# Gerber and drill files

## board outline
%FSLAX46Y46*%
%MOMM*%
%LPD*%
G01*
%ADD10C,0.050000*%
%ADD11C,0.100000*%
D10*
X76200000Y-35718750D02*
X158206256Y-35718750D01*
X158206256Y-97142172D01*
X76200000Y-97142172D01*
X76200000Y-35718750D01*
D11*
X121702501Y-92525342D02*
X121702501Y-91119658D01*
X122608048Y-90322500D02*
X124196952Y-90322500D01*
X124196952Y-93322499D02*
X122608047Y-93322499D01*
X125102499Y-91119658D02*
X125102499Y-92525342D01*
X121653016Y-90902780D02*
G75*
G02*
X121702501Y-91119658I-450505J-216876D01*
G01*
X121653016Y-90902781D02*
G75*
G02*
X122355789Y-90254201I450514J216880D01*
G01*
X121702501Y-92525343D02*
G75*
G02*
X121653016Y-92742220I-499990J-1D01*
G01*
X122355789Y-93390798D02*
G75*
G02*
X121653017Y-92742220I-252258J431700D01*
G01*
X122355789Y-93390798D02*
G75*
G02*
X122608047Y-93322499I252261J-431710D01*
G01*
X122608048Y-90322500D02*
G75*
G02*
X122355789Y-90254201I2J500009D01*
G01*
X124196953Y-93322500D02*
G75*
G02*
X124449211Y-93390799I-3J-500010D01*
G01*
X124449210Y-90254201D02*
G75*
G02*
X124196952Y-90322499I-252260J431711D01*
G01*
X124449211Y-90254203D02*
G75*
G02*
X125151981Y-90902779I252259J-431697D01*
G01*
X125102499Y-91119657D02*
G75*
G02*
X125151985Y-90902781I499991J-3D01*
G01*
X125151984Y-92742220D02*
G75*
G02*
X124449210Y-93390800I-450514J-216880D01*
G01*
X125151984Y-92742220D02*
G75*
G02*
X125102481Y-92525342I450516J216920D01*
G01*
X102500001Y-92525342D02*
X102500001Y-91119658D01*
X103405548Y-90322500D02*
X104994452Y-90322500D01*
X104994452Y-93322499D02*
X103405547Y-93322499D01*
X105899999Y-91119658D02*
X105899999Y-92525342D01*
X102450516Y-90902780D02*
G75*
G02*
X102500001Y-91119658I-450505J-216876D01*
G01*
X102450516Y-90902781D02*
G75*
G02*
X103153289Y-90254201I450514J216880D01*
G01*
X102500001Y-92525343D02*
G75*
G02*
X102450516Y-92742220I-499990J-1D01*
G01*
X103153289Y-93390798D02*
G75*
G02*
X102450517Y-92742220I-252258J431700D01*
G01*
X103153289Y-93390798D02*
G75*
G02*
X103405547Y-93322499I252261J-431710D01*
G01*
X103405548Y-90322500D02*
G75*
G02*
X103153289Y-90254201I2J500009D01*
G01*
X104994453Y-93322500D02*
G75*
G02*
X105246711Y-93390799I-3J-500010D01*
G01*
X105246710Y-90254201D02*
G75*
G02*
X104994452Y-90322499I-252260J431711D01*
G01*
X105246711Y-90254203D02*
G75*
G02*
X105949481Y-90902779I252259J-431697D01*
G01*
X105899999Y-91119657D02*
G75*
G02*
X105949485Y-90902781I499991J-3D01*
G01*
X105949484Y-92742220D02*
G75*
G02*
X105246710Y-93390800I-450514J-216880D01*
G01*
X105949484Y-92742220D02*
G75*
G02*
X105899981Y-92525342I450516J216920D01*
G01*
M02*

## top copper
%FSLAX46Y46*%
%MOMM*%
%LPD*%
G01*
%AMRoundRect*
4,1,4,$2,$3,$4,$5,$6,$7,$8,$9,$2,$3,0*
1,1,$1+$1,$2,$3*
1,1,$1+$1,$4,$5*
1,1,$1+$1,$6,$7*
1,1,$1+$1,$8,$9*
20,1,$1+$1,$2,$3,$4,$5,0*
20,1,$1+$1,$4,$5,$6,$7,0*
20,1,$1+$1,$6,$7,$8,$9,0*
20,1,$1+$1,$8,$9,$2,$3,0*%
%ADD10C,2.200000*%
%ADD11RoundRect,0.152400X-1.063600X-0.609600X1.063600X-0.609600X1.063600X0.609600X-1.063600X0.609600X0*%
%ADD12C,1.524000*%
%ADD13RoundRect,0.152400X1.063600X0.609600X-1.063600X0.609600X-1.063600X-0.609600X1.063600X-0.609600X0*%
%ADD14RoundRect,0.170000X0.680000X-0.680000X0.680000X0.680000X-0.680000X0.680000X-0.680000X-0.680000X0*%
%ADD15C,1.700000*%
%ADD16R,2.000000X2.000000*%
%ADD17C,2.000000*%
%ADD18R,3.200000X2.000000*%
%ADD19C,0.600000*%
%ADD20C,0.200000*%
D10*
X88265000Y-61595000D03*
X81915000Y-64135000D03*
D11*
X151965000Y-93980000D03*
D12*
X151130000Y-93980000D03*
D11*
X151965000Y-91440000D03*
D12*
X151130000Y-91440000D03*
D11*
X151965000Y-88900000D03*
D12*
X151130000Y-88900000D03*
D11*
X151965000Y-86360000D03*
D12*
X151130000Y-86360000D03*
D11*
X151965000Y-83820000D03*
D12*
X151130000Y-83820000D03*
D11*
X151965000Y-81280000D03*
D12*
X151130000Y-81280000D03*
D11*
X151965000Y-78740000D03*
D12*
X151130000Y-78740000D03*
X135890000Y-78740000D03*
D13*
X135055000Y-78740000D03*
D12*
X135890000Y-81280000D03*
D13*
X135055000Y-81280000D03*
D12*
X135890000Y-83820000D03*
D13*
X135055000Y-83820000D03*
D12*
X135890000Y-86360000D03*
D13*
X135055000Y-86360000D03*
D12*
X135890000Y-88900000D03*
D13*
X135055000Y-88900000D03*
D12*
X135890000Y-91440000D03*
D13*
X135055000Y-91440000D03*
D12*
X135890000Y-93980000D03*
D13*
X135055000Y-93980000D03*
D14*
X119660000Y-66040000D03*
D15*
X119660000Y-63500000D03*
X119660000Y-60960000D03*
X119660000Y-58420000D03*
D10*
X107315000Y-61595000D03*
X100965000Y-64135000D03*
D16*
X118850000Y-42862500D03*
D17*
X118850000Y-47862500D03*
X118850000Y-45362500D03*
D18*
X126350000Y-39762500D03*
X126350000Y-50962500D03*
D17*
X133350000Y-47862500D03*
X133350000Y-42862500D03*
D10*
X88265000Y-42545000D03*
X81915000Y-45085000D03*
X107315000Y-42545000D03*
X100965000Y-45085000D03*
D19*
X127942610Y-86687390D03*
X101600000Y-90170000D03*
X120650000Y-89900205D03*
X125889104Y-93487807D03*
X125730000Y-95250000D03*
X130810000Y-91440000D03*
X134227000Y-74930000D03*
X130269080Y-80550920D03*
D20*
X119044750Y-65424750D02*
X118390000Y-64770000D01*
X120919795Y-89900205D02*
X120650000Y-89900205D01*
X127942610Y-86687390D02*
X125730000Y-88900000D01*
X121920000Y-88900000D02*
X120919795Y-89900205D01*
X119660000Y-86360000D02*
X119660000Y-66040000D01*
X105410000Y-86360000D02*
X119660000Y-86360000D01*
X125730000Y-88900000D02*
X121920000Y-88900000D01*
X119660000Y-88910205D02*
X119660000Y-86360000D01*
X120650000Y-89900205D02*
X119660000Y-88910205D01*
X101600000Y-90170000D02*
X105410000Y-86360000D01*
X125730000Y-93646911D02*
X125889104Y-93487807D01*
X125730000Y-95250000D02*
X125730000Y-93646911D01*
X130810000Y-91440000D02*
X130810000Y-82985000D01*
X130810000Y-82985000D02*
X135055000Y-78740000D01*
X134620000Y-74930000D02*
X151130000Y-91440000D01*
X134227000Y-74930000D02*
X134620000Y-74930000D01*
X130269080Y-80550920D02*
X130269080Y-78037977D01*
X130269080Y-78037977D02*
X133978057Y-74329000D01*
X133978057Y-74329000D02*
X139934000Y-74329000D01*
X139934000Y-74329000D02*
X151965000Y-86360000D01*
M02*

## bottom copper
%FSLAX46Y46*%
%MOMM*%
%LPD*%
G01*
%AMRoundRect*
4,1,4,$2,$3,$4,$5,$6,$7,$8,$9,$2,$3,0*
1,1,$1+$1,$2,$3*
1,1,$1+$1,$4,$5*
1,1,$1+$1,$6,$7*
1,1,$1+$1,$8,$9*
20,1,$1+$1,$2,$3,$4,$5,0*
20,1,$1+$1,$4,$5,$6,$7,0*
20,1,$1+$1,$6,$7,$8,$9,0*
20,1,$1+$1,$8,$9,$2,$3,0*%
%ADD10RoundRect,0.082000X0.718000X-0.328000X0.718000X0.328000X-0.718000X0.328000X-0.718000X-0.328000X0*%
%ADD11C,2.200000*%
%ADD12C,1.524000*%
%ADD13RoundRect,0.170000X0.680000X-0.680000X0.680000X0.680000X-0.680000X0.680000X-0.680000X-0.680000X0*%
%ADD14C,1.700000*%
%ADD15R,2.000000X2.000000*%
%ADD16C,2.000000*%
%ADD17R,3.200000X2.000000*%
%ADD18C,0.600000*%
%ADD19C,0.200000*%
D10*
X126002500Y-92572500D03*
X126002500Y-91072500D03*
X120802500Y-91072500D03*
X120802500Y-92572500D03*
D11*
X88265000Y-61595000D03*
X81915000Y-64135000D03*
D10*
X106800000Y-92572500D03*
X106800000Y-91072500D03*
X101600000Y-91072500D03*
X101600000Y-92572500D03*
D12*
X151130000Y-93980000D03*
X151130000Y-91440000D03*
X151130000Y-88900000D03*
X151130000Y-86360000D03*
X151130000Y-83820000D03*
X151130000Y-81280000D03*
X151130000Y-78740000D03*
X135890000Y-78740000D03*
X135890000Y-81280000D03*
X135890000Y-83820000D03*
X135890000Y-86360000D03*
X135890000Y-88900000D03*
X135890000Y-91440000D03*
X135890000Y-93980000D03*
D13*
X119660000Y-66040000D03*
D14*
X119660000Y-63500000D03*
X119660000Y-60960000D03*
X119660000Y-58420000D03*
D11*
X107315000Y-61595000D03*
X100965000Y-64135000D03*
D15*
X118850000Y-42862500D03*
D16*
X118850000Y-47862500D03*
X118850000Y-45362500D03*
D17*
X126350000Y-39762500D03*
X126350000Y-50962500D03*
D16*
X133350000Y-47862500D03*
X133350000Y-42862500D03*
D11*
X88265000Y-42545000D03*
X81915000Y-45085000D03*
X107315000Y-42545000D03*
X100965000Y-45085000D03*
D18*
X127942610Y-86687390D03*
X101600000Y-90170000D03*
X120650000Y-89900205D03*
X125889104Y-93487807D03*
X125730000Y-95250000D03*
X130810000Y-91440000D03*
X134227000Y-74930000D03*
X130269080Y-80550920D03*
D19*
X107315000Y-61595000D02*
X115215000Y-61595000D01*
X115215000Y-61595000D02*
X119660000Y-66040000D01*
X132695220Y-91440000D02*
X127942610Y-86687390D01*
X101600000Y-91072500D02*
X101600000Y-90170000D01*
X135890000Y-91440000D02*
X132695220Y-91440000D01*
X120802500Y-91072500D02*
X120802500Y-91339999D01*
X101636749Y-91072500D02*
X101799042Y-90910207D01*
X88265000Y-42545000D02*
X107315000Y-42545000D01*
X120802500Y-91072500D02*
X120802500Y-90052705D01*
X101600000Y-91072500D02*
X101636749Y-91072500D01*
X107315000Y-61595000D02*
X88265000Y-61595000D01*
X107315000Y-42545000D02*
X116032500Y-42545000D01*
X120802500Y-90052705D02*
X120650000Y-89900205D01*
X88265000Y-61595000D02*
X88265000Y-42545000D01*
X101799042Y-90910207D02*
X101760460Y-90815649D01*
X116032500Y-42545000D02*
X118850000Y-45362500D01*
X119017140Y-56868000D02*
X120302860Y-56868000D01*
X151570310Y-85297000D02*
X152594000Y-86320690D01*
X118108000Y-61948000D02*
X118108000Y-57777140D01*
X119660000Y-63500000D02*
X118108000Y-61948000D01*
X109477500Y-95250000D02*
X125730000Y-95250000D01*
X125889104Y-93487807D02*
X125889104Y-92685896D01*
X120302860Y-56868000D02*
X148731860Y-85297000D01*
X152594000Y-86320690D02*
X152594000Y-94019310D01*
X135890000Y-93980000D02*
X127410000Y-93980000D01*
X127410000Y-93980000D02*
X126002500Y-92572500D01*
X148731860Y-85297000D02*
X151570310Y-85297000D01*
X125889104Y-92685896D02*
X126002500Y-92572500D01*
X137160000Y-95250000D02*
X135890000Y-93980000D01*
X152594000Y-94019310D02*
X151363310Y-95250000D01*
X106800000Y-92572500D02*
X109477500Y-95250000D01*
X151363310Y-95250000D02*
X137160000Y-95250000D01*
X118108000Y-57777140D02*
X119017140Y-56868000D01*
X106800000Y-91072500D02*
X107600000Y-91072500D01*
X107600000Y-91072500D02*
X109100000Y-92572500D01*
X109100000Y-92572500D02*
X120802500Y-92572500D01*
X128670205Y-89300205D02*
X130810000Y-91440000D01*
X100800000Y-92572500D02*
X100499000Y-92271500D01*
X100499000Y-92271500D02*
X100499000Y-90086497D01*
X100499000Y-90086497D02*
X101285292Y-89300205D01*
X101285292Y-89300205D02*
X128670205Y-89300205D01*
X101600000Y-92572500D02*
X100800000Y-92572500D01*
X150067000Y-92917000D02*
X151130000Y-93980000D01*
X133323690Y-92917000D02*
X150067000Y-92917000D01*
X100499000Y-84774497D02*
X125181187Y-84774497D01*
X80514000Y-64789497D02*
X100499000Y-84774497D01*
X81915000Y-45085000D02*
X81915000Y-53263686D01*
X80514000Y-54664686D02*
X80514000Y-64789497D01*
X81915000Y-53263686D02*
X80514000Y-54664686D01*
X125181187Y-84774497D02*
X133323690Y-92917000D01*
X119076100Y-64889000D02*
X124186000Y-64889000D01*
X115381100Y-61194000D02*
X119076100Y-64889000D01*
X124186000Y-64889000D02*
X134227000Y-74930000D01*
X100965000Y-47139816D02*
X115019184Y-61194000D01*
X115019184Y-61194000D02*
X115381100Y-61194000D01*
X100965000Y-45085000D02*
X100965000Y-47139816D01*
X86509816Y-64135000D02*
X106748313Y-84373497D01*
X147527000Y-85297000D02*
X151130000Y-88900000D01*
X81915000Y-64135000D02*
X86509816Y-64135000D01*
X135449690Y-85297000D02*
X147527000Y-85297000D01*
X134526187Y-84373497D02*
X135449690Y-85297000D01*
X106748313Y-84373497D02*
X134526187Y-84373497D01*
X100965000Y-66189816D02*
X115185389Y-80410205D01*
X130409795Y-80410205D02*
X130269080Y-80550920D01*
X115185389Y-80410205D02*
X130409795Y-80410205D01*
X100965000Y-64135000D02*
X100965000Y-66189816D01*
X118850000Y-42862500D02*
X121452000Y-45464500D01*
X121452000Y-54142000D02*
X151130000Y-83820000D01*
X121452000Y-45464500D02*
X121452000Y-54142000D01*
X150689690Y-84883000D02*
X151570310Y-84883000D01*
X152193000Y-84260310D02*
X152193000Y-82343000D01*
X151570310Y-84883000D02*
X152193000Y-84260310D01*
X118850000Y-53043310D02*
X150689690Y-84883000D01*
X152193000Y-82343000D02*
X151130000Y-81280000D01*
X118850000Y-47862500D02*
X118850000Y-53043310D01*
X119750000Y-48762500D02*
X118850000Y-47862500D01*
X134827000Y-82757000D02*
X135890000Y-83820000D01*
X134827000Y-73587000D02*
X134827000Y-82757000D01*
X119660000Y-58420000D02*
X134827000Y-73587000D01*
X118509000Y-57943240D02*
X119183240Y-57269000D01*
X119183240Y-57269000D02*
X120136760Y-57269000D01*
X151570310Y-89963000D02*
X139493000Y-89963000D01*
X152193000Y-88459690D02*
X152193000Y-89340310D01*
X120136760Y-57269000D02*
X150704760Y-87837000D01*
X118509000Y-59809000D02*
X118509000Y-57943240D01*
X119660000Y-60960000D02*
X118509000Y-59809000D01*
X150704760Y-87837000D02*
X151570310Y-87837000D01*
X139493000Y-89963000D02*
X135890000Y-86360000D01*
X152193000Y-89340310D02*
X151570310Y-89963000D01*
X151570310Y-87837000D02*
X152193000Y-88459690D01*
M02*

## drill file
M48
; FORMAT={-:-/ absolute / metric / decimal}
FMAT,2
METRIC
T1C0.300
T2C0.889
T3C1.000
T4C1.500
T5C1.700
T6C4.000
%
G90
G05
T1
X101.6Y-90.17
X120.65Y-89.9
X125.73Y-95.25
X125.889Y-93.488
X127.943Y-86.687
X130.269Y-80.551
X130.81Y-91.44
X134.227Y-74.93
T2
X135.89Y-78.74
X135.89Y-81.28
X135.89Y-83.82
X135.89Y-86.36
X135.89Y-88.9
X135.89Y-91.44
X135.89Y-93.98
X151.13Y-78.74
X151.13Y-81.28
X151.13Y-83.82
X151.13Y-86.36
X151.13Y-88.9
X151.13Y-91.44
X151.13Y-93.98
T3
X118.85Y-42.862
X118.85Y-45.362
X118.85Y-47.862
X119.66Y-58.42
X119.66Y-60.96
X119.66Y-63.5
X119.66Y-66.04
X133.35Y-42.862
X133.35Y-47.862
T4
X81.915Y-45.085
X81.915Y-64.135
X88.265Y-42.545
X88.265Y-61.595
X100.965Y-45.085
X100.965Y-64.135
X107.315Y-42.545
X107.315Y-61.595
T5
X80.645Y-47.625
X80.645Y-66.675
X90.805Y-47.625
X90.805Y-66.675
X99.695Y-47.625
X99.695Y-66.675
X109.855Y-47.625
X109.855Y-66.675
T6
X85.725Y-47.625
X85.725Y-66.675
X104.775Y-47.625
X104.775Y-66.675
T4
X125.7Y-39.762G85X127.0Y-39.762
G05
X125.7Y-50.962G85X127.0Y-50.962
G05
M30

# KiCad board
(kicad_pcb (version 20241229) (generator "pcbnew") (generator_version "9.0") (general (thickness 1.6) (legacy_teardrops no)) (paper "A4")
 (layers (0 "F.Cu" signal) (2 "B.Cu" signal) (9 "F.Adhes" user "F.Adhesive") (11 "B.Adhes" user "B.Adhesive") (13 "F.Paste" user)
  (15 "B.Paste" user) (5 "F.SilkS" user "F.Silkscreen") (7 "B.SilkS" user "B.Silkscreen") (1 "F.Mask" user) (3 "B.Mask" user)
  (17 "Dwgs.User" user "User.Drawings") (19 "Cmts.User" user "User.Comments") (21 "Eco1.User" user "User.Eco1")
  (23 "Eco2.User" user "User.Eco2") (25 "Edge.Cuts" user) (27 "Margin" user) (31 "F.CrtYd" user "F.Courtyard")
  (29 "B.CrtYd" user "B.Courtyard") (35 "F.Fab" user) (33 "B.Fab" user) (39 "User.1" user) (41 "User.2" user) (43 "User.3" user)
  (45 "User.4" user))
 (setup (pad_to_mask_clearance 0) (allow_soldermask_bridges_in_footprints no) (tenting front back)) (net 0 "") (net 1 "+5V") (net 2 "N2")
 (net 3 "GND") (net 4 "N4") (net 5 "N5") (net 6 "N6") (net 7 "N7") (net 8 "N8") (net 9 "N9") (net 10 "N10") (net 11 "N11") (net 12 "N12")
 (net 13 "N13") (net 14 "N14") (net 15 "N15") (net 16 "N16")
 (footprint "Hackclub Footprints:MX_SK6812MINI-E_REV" (layer "F.Cu") (at 123.4025 86.7425)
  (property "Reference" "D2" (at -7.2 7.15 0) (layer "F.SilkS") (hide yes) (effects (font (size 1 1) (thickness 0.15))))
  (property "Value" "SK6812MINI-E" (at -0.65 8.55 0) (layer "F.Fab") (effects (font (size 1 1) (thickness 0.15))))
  (fp_line (start -1.699999 5.782842) (end -1.699999 4.377158) (stroke (width 0.1) (type solid)) (layer "Edge.Cuts"))
  (fp_line (start -0.794452 3.58) (end 0.794452 3.58) (stroke (width 0.1) (type solid)) (layer "Edge.Cuts"))
  (fp_line (start 0.794452 6.579999) (end -0.794453 6.579999) (stroke (width 0.1) (type solid)) (layer "Edge.Cuts"))
  (fp_line (start 1.699999 4.377158) (end 1.699999 5.782842) (stroke (width 0.1) (type solid)) (layer "Edge.Cuts"))
  (fp_arc (start -1.749484 4.16028) (mid -1.712527 4.265932) (end -1.699999 4.377158) (stroke (width 0.1) (type solid)) (layer "Edge.Cuts"))
  (fp_arc (start -1.749484 4.160281) (mid -1.638072 3.575965) (end -1.046711 3.511701) (stroke (width 0.1) (type solid)) (layer "Edge.Cuts"))
  (fp_arc (start -1.699999 5.782843) (mid -1.712527 5.894068) (end -1.749484 5.99972) (stroke (width 0.1) (type solid)) (layer "Edge.Cuts"))
  (fp_arc (start -1.046711 6.648298) (mid -1.638071 6.584034) (end -1.749484 5.99972) (stroke (width 0.1) (type solid)) (layer "Edge.Cuts"))
  (fp_arc (start -1.046711 6.648298) (mid -0.925123 6.597376) (end -0.794453 6.579999) (stroke (width 0.1) (type solid)) (layer "Edge.Cuts"))
  (fp_arc (start -0.794452 3.58) (mid -0.925123 3.562623) (end -1.046711 3.511701) (stroke (width 0.1) (type solid)) (layer "Edge.Cuts"))
  (fp_arc (start 0.794453 6.58) (mid 0.925123 6.597377) (end 1.046711 6.648299) (stroke (width 0.1) (type solid)) (layer "Edge.Cuts"))
  (fp_arc (start 1.04671 3.511701) (mid 0.925122 3.562623) (end 0.794452 3.58) (stroke (width 0.1) (type solid)) (layer "Edge.Cuts"))
  (fp_arc (start 1.046711 3.511703) (mid 1.63807 3.575966) (end 1.749484 4.16028) (stroke (width 0.1) (type solid)) (layer "Edge.Cuts"))
  (fp_arc (start 1.699999 4.377157) (mid 1.712527 4.265932) (end 1.749484 4.16028) (stroke (width 0.1) (type solid)) (layer "Edge.Cuts"))
  (fp_arc (start 1.749484 5.99972) (mid 1.638071 6.584035) (end 1.046711 6.648299) (stroke (width 0.1) (type solid)) (layer "Edge.Cuts"))
  (fp_arc (start 1.749484 5.99972) (mid 1.712527 5.894068) (end 1.699999 5.782842) (stroke (width 0.1) (type solid)) (layer "Edge.Cuts"))
  (pad "1" smd roundrect (at 2.6 5.83 90) (size 0.82 1.6) (layers "B.Cu" "B.Mask" "B.Paste") (roundrect_rratio 0.1) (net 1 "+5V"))
  (pad "2" smd roundrect (at 2.6 4.33 90) (size 0.82 1.6) (layers "B.Cu" "B.Mask" "B.Paste") (roundrect_rratio 0.1) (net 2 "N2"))
  (pad "3" smd roundrect (at -2.6 4.33 90) (size 0.82 1.6) (layers "B.Cu" "B.Mask" "B.Paste") (roundrect_rratio 0.1) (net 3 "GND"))
  (pad "4" smd roundrect (at -2.6 5.83 90) (size 0.82 1.6) (layers "B.Cu" "B.Mask" "B.Paste") (roundrect_rratio 0.1) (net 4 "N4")))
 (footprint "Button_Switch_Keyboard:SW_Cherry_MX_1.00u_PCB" (layer "F.Cu") (at 88.265 61.595)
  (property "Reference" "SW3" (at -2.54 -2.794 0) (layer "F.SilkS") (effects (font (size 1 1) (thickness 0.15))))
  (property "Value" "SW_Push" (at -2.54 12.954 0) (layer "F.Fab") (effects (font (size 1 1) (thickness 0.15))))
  (pad "" np_thru_hole circle (at -7.62 5.08) (size 1.7 1.7) (drill 1.7) (layers "*.Cu" "*.Mask"))
  (pad "" np_thru_hole circle (at -2.54 5.08) (size 4 4) (drill 4) (layers "*.Cu" "*.Mask"))
  (pad "" np_thru_hole circle (at 2.54 5.08) (size 1.7 1.7) (drill 1.7) (layers "*.Cu" "*.Mask"))
  (pad "1" thru_hole circle (at 0 0) (size 2.2 2.2) (drill 1.5) (layers "*.Cu" "*.Mask") (remove_unused_layers no) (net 3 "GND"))
  (pad "2" thru_hole circle (at -6.35 2.54) (size 2.2 2.2) (drill 1.5) (layers "*.Cu" "*.Mask") (remove_unused_layers no) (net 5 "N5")))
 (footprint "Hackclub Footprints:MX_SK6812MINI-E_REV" (layer "F.Cu") (at 104.2 86.7425)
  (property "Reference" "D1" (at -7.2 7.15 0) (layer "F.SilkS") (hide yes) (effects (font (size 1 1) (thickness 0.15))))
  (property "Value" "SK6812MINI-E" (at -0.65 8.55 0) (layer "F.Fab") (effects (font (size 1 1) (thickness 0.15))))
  (fp_line (start -1.699999 5.782842) (end -1.699999 4.377158) (stroke (width 0.1) (type solid)) (layer "Edge.Cuts"))
  (fp_line (start -0.794452 3.58) (end 0.794452 3.58) (stroke (width 0.1) (type solid)) (layer "Edge.Cuts"))
  (fp_line (start 0.794452 6.579999) (end -0.794453 6.579999) (stroke (width 0.1) (type solid)) (layer "Edge.Cuts"))
  (fp_line (start 1.699999 4.377158) (end 1.699999 5.782842) (stroke (width 0.1) (type solid)) (layer "Edge.Cuts"))
  (fp_arc (start -1.749484 4.16028) (mid -1.712527 4.265932) (end -1.699999 4.377158) (stroke (width 0.1) (type solid)) (layer "Edge.Cuts"))
  (fp_arc (start -1.749484 4.160281) (mid -1.638072 3.575965) (end -1.046711 3.511701) (stroke (width 0.1) (type solid)) (layer "Edge.Cuts"))
  (fp_arc (start -1.699999 5.782843) (mid -1.712527 5.894068) (end -1.749484 5.99972) (stroke (width 0.1) (type solid)) (layer "Edge.Cuts"))
  (fp_arc (start -1.046711 6.648298) (mid -1.638071 6.584034) (end -1.749484 5.99972) (stroke (width 0.1) (type solid)) (layer "Edge.Cuts"))
  (fp_arc (start -1.046711 6.648298) (mid -0.925123 6.597376) (end -0.794453 6.579999) (stroke (width 0.1) (type solid)) (layer "Edge.Cuts"))
  (fp_arc (start -0.794452 3.58) (mid -0.925123 3.562623) (end -1.046711 3.511701) (stroke (width 0.1) (type solid)) (layer "Edge.Cuts"))
  (fp_arc (start 0.794453 6.58) (mid 0.925123 6.597377) (end 1.046711 6.648299) (stroke (width 0.1) (type solid)) (layer "Edge.Cuts"))
  (fp_arc (start 1.04671 3.511701) (mid 0.925122 3.562623) (end 0.794452 3.58) (stroke (width 0.1) (type solid)) (layer "Edge.Cuts"))
  (fp_arc (start 1.046711 3.511703) (mid 1.63807 3.575966) (end 1.749484 4.16028) (stroke (width 0.1) (type solid)) (layer "Edge.Cuts"))
  (fp_arc (start 1.699999 4.377157) (mid 1.712527 4.265932) (end 1.749484 4.16028) (stroke (width 0.1) (type solid)) (layer "Edge.Cuts"))
  (fp_arc (start 1.749484 5.99972) (mid 1.638071 6.584035) (end 1.046711 6.648299) (stroke (width 0.1) (type solid)) (layer "Edge.Cuts"))
  (fp_arc (start 1.749484 5.99972) (mid 1.712527 5.894068) (end 1.699999 5.782842) (stroke (width 0.1) (type solid)) (layer "Edge.Cuts"))
  (pad "1" smd roundrect (at 2.6 5.83 90) (size 0.82 1.6) (layers "B.Cu" "B.Mask" "B.Paste") (roundrect_rratio 0.1) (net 1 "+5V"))
  (pad "2" smd roundrect (at 2.6 4.33 90) (size 0.82 1.6) (layers "B.Cu" "B.Mask" "B.Paste") (roundrect_rratio 0.1) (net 4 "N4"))
  (pad "3" smd roundrect (at -2.6 4.33 90) (size 0.82 1.6) (layers "B.Cu" "B.Mask" "B.Paste") (roundrect_rratio 0.1) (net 3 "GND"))
  (pad "4" smd roundrect (at -2.6 5.83 90) (size 0.82 1.6) (layers "B.Cu" "B.Mask" "B.Paste") (roundrect_rratio 0.1) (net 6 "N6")))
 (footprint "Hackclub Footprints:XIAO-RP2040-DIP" (layer "F.Cu") (at 143.51 86.36 180)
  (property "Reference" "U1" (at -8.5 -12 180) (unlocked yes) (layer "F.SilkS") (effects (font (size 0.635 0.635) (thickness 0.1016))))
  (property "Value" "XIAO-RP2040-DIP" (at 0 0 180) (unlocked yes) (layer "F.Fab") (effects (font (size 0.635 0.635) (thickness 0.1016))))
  (pad "1" smd roundrect (at -8.455 -7.62) (size 2.432 1.524) (layers "F.Cu" "F.Mask") (roundrect_rratio 0.1) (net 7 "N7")
   (thermal_bridge_angle 45))
  (pad "1" thru_hole circle (at -7.62 -7.62) (size 1.524 1.524) (drill 0.889) (layers "*.Cu" "*.Mask") (remove_unused_layers no)
   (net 7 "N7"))
  (pad "2" smd roundrect (at -8.455 -5.08) (size 2.432 1.524) (layers "F.Cu" "F.Mask") (roundrect_rratio 0.1) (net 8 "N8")
   (thermal_bridge_angle 45))
  (pad "2" thru_hole circle (at -7.62 -5.08) (size 1.524 1.524) (drill 0.889) (layers "*.Cu" "*.Mask") (remove_unused_layers no)
   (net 8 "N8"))
  (pad "3" smd roundrect (at -8.455 -2.54) (size 2.432 1.524) (layers "F.Cu" "F.Mask") (roundrect_rratio 0.1) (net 5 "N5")
   (thermal_bridge_angle 45))
  (pad "3" thru_hole circle (at -7.62 -2.54) (size 1.524 1.524) (drill 0.889) (layers "*.Cu" "*.Mask") (remove_unused_layers no)
   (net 5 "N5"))
  (pad "4" smd roundrect (at -8.455 0) (size 2.432 1.524) (layers "F.Cu" "F.Mask") (roundrect_rratio 0.1) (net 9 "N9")
   (thermal_bridge_angle 45))
  (pad "4" thru_hole circle (at -7.62 0) (size 1.524 1.524) (drill 0.889) (layers "*.Cu" "*.Mask") (remove_unused_layers no) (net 9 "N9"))
  (pad "5" smd roundrect (at -8.455 2.54) (size 2.432 1.524) (layers "F.Cu" "F.Mask") (roundrect_rratio 0.1) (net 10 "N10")
   (thermal_bridge_angle 45))
  (pad "5" thru_hole circle (at -7.62 2.54) (size 1.524 1.524) (drill 0.889) (layers "*.Cu" "*.Mask") (remove_unused_layers no)
   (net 10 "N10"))
  (pad "6" smd roundrect (at -8.455 5.08) (size 2.432 1.524) (layers "F.Cu" "F.Mask") (roundrect_rratio 0.1) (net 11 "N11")
   (thermal_bridge_angle 45))
  (pad "6" thru_hole circle (at -7.62 5.08) (size 1.524 1.524) (drill 0.889) (layers "*.Cu" "*.Mask") (remove_unused_layers no)
   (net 11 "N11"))
  (pad "7" smd roundrect (at -8.455 7.62) (size 2.432 1.524) (layers "F.Cu" "F.Mask") (roundrect_rratio 0.1) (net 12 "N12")
   (thermal_bridge_angle 45))
  (pad "7" thru_hole circle (at -7.62 7.62) (size 1.524 1.524) (drill 0.889) (layers "*.Cu" "*.Mask") (remove_unused_layers no)
   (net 12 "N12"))
  (pad "8" thru_hole circle (at 7.62 7.62 180) (size 1.524 1.524) (drill 0.889) (layers "*.Cu" "*.Mask") (remove_unused_layers no)
   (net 6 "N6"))
  (pad "8" smd roundrect (at 8.455 7.62 180) (size 2.432 1.524) (layers "F.Cu" "F.Mask") (roundrect_rratio 0.1) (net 6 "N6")
   (thermal_bridge_angle 45))
  (pad "9" thru_hole circle (at 7.62 5.08 180) (size 1.524 1.524) (drill 0.889) (layers "*.Cu" "*.Mask") (remove_unused_layers no)
   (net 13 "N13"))
  (pad "9" smd roundrect (at 8.455 5.08 180) (size 2.432 1.524) (layers "F.Cu" "F.Mask") (roundrect_rratio 0.1) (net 13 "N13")
   (thermal_bridge_angle 45))
  (pad "10" thru_hole circle (at 7.62 2.54 180) (size 1.524 1.524) (drill 0.889) (layers "*.Cu" "*.Mask") (remove_unused_layers no)
   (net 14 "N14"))
  (pad "10" smd roundrect (at 8.455 2.54 180) (size 2.432 1.524) (layers "F.Cu" "F.Mask") (roundrect_rratio 0.1) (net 14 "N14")
   (thermal_bridge_angle 45))
  (pad "11" thru_hole circle (at 7.62 0 180) (size 1.524 1.524) (drill 0.889) (layers "*.Cu" "*.Mask") (remove_unused_layers no)
   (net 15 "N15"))
  (pad "11" smd roundrect (at 8.455 0 180) (size 2.432 1.524) (layers "F.Cu" "F.Mask") (roundrect_rratio 0.1) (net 15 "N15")
   (thermal_bridge_angle 45))
  (pad "12" thru_hole circle (at 7.62 -2.54 180) (size 1.524 1.524) (drill 0.889) (layers "*.Cu" "*.Mask") (remove_unused_layers no)
   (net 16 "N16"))
  (pad "12" smd roundrect (at 8.455 -2.54 180) (size 2.432 1.524) (layers "F.Cu" "F.Mask") (roundrect_rratio 0.1) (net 16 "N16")
   (thermal_bridge_angle 45))
  (pad "13" thru_hole circle (at 7.62 -5.08 180) (size 1.524 1.524) (drill 0.889) (layers "*.Cu" "*.Mask") (remove_unused_layers no)
   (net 3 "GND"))
  (pad "13" smd roundrect (at 8.455 -5.08 180) (size 2.432 1.524) (layers "F.Cu" "F.Mask") (roundrect_rratio 0.1) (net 3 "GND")
   (thermal_bridge_angle 45))
  (pad "14" thru_hole circle (at 7.62 -7.62 180) (size 1.524 1.524) (drill 0.889) (layers "*.Cu" "*.Mask") (remove_unused_layers no)
   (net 1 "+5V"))
  (pad "14" smd roundrect (at 8.455 -7.62 180) (size 2.432 1.524) (layers "F.Cu" "F.Mask") (roundrect_rratio 0.1) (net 1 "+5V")
   (thermal_bridge_angle 45)))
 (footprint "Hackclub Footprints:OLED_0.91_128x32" (layer "F.Cu") (at 119.66 66.04 90)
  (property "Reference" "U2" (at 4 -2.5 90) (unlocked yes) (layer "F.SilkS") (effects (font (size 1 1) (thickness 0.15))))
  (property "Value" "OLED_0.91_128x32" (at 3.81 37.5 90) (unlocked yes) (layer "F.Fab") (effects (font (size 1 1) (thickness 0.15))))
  (pad "1" thru_hole roundrect (at 0 0 90) (size 1.7 1.7) (drill 1) (layers "*.Cu" "*.Mask") (remove_unused_layers no)
   (roundrect_rratio 0.1) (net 3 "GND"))
  (pad "2" thru_hole circle (at 2.54 0 90) (size 1.7 1.7) (drill 1) (layers "*.Cu" "*.Mask") (remove_unused_layers no) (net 1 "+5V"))
  (pad "3" thru_hole circle (at 5.08 0 90) (size 1.7 1.7) (drill 1) (layers "*.Cu" "*.Mask") (remove_unused_layers no) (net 15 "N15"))
  (pad "4" thru_hole circle (at 7.62 0 90) (size 1.7 1.7) (drill 1) (layers "*.Cu" "*.Mask") (remove_unused_layers no) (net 14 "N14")))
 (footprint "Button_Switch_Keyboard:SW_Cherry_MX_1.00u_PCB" (layer "F.Cu") (at 107.315 61.595)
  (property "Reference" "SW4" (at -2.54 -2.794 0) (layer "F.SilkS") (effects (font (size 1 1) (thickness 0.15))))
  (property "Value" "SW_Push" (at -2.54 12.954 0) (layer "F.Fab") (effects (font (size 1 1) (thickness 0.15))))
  (pad "" np_thru_hole circle (at -7.62 5.08) (size 1.7 1.7) (drill 1.7) (layers "*.Cu" "*.Mask"))
  (pad "" np_thru_hole circle (at -2.54 5.08) (size 4 4) (drill 4) (layers "*.Cu" "*.Mask"))
  (pad "" np_thru_hole circle (at 2.54 5.08) (size 1.7 1.7) (drill 1.7) (layers "*.Cu" "*.Mask"))
  (pad "1" thru_hole circle (at 0 0) (size 2.2 2.2) (drill 1.5) (layers "*.Cu" "*.Mask") (remove_unused_layers no) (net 3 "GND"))
  (pad "2" thru_hole circle (at -6.35 2.54) (size 2.2 2.2) (drill 1.5) (layers "*.Cu" "*.Mask") (remove_unused_layers no) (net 9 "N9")))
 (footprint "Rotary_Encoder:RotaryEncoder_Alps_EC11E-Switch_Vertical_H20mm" (layer "F.Cu") (at 118.85 42.8625)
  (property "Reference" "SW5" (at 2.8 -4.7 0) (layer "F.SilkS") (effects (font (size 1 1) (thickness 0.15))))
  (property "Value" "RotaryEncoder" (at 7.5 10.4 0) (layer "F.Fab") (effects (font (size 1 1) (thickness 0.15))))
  (pad "A" thru_hole rect (at 0 0) (size 2 2) (drill 1) (layers "*.Cu" "*.Mask") (remove_unused_layers no) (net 10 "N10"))
  (pad "B" thru_hole circle (at 0 5) (size 2 2) (drill 1) (layers "*.Cu" "*.Mask") (remove_unused_layers no) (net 11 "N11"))
  (pad "C" thru_hole circle (at 0 2.5) (size 2 2) (drill 1) (layers "*.Cu" "*.Mask") (remove_unused_layers no) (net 3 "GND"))
  (pad "MP" thru_hole rect (at 7.5 -3.1) (size 3.2 2) (drill oval 2.8 1.5) (layers "*.Cu" "*.Mask") (remove_unused_layers no))
  (pad "MP" thru_hole rect (at 7.5 8.1) (size 3.2 2) (drill oval 2.8 1.5) (layers "*.Cu" "*.Mask") (remove_unused_layers no))
  (pad "S1" thru_hole circle (at 14.5 5) (size 2 2) (drill 1) (layers "*.Cu" "*.Mask") (remove_unused_layers no))
  (pad "S2" thru_hole circle (at 14.5 0) (size 2 2) (drill 1) (layers "*.Cu" "*.Mask") (remove_unused_layers no)))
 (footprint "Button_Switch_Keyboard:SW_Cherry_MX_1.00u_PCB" (layer "F.Cu") (at 88.265 42.545)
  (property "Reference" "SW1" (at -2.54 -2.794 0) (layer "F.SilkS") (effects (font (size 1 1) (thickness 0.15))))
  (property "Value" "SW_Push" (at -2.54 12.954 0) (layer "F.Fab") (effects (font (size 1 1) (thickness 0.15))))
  (pad "" np_thru_hole circle (at -7.62 5.08) (size 1.7 1.7) (drill 1.7) (layers "*.Cu" "*.Mask"))
  (pad "" np_thru_hole circle (at -2.54 5.08) (size 4 4) (drill 4) (layers "*.Cu" "*.Mask"))
  (pad "" np_thru_hole circle (at 2.54 5.08) (size 1.7 1.7) (drill 1.7) (layers "*.Cu" "*.Mask"))
  (pad "1" thru_hole circle (at 0 0) (size 2.2 2.2) (drill 1.5) (layers "*.Cu" "*.Mask") (remove_unused_layers no) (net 3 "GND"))
  (pad "2" thru_hole circle (at -6.35 2.54) (size 2.2 2.2) (drill 1.5) (layers "*.Cu" "*.Mask") (remove_unused_layers no) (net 7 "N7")))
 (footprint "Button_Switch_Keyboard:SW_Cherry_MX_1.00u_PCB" (layer "F.Cu") (at 107.315 42.545)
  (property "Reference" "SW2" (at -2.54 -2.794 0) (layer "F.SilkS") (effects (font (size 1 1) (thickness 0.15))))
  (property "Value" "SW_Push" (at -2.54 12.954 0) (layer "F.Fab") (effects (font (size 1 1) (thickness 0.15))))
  (pad "" np_thru_hole circle (at -7.62 5.08) (size 1.7 1.7) (drill 1.7) (layers "*.Cu" "*.Mask"))
  (pad "" np_thru_hole circle (at -2.54 5.08) (size 4 4) (drill 4) (layers "*.Cu" "*.Mask"))
  (pad "" np_thru_hole circle (at 2.54 5.08) (size 1.7 1.7) (drill 1.7) (layers "*.Cu" "*.Mask"))
  (pad "1" thru_hole circle (at 0 0) (size 2.2 2.2) (drill 1.5) (layers "*.Cu" "*.Mask") (remove_unused_layers no) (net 3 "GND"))
  (pad "2" thru_hole circle (at -6.35 2.54) (size 2.2 2.2) (drill 1.5) (layers "*.Cu" "*.Mask") (remove_unused_layers no) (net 8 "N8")))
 (gr_rect (start 76.2 35.71875) (end 158.206256 97.142172) (stroke (width 0.05) (type default)) (fill no) (layer "Edge.Cuts"))
 (segment (start 119.04475 65.42475) (end 118.39 64.77) (width 0.2) (layer "F.Cu") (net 3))
 (segment (start 120.919795 89.900205) (end 120.65 89.900205) (width 0.2) (layer "F.Cu") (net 3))
 (segment (start 127.94261 86.68739) (end 125.73 88.9) (width 0.2) (layer "F.Cu") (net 3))
 (segment (start 121.92 88.9) (end 120.919795 89.900205) (width 0.2) (layer "F.Cu") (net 3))
 (segment (start 119.66 86.36) (end 119.66 66.04) (width 0.2) (layer "F.Cu") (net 3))
 (segment (start 105.41 86.36) (end 119.66 86.36) (width 0.2) (layer "F.Cu") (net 3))
 (segment (start 125.73 88.9) (end 121.92 88.9) (width 0.2) (layer "F.Cu") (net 3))
 (segment (start 119.66 88.910205) (end 119.66 86.36) (width 0.2) (layer "F.Cu") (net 3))
 (segment (start 120.65 89.900205) (end 119.66 88.910205) (width 0.2) (layer "F.Cu") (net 3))
 (segment (start 101.6 90.17) (end 105.41 86.36) (width 0.2) (layer "F.Cu") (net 3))
 (via (at 127.94261 86.68739) (size 0.6) (drill 0.3) (layers "F.Cu" "B.Cu") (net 3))
 (via (at 101.6 90.17) (size 0.6) (drill 0.3) (layers "F.Cu" "B.Cu") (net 3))
 (via (at 120.65 89.900205) (size 0.6) (drill 0.3) (layers "F.Cu" "B.Cu") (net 3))
 (segment (start 107.315 61.595) (end 115.215 61.595) (width 0.2) (layer "B.Cu") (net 3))
 (segment (start 115.215 61.595) (end 119.66 66.04) (width 0.2) (layer "B.Cu") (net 3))
 (segment (start 132.69522 91.44) (end 127.94261 86.68739) (width 0.2) (layer "B.Cu") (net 3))
 (segment (start 101.6 91.0725) (end 101.6 90.17) (width 0.2) (layer "B.Cu") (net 3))
 (segment (start 135.89 91.44) (end 132.69522 91.44) (width 0.2) (layer "B.Cu") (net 3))
 (segment (start 120.8025 91.0725) (end 120.8025 91.339999) (width 0.2) (layer "B.Cu") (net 3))
 (segment (start 101.636749 91.0725) (end 101.799042 90.910207) (width 0.2) (layer "B.Cu") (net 3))
 (segment (start 88.265 42.545) (end 107.315 42.545) (width 0.2) (layer "B.Cu") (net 3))
 (segment (start 120.8025 91.0725) (end 120.8025 90.052705) (width 0.2) (layer "B.Cu") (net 3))
 (segment (start 101.6 91.0725) (end 101.636749 91.0725) (width 0.2) (layer "B.Cu") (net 3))
 (segment (start 107.315 61.595) (end 88.265 61.595) (width 0.2) (layer "B.Cu") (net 3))
 (segment (start 107.315 42.545) (end 116.0325 42.545) (width 0.2) (layer "B.Cu") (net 3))
 (segment (start 120.8025 90.052705) (end 120.65 89.900205) (width 0.2) (layer "B.Cu") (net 3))
 (segment (start 88.265 61.595) (end 88.265 42.545) (width 0.2) (layer "B.Cu") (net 3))
 (segment (start 101.799042 90.910207) (end 101.76046 90.815649) (width 0.2) (layer "B.Cu") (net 3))
 (segment (start 116.0325 42.545) (end 118.85 45.3625) (width 0.2) (layer "B.Cu") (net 3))
 (segment (start 125.73 93.646911) (end 125.889104 93.487807) (width 0.2) (layer "F.Cu") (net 1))
 (segment (start 125.73 95.25) (end 125.73 93.646911) (width 0.2) (layer "F.Cu") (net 1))
 (via (at 125.889104 93.487807) (size 0.6) (drill 0.3) (layers "F.Cu" "B.Cu") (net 1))
 (via (at 125.73 95.25) (size 0.6) (drill 0.3) (layers "F.Cu" "B.Cu") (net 1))
 (segment (start 119.01714 56.868) (end 120.30286 56.868) (width 0.2) (layer "B.Cu") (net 1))
 (segment (start 151.57031 85.297) (end 152.594 86.32069) (width 0.2) (layer "B.Cu") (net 1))
 (segment (start 118.108 61.948) (end 118.108 57.77714) (width 0.2) (layer "B.Cu") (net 1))
 (segment (start 119.66 63.5) (end 118.108 61.948) (width 0.2) (layer "B.Cu") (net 1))
 (segment (start 109.4775 95.25) (end 125.73 95.25) (width 0.2) (layer "B.Cu") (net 1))
 (segment (start 125.889104 93.487807) (end 125.889104 92.685896) (width 0.2) (layer "B.Cu") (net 1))
 (segment (start 120.30286 56.868) (end 148.73186 85.297) (width 0.2) (layer "B.Cu") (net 1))
 (segment (start 152.594 86.32069) (end 152.594 94.01931) (width 0.2) (layer "B.Cu") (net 1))
 (segment (start 135.89 93.98) (end 127.41 93.98) (width 0.2) (layer "B.Cu") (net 1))
 (segment (start 127.41 93.98) (end 126.0025 92.5725) (width 0.2) (layer "B.Cu") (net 1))
 (segment (start 148.73186 85.297) (end 151.57031 85.297) (width 0.2) (layer "B.Cu") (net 1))
 (segment (start 125.889104 92.685896) (end 126.0025 92.5725) (width 0.2) (layer "B.Cu") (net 1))
 (segment (start 137.16 95.25) (end 135.89 93.98) (width 0.2) (layer "B.Cu") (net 1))
 (segment (start 152.594 94.01931) (end 151.36331 95.25) (width 0.2) (layer "B.Cu") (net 1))
 (segment (start 106.8 92.5725) (end 109.4775 95.25) (width 0.2) (layer "B.Cu") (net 1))
 (segment (start 151.36331 95.25) (end 137.16 95.25) (width 0.2) (layer "B.Cu") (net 1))
 (segment (start 118.108 57.77714) (end 119.01714 56.868) (width 0.2) (layer "B.Cu") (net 1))
 (segment (start 106.8 91.0725) (end 107.6 91.0725) (width 0.2) (layer "B.Cu") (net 4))
 (segment (start 107.6 91.0725) (end 109.1 92.5725) (width 0.2) (layer "B.Cu") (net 4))
 (segment (start 109.1 92.5725) (end 120.8025 92.5725) (width 0.2) (layer "B.Cu") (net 4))
 (segment (start 130.81 91.44) (end 130.81 82.985) (width 0.2) (layer "F.Cu") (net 6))
 (segment (start 130.81 82.985) (end 135.055 78.74) (width 0.2) (layer "F.Cu") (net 6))
 (via (at 130.81 91.44) (size 0.6) (drill 0.3) (layers "F.Cu" "B.Cu") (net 6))
 (segment (start 128.670205 89.300205) (end 130.81 91.44) (width 0.2) (layer "B.Cu") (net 6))
 (segment (start 100.8 92.5725) (end 100.499 92.2715) (width 0.2) (layer "B.Cu") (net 6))
 (segment (start 100.499 92.2715) (end 100.499 90.086497) (width 0.2) (layer "B.Cu") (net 6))
 (segment (start 100.499 90.086497) (end 101.285292 89.300205) (width 0.2) (layer "B.Cu") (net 6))
 (segment (start 101.285292 89.300205) (end 128.670205 89.300205) (width 0.2) (layer "B.Cu") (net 6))
 (segment (start 101.6 92.5725) (end 100.8 92.5725) (width 0.2) (layer "B.Cu") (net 6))
 (segment (start 150.067 92.917) (end 151.13 93.98) (width 0.2) (layer "B.Cu") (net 7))
 (segment (start 133.32369 92.917) (end 150.067 92.917) (width 0.2) (layer "B.Cu") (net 7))
 (segment (start 100.499 84.774497) (end 125.181187 84.774497) (width 0.2) (layer "B.Cu") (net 7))
 (segment (start 80.514 64.789497) (end 100.499 84.774497) (width 0.2) (layer "B.Cu") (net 7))
 (segment (start 81.915 45.085) (end 81.915 53.263686) (width 0.2) (layer "B.Cu") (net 7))
 (segment (start 80.514 54.664686) (end 80.514 64.789497) (width 0.2) (layer "B.Cu") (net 7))
 (segment (start 81.915 53.263686) (end 80.514 54.664686) (width 0.2) (layer "B.Cu") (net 7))
 (segment (start 125.181187 84.774497) (end 133.32369 92.917) (width 0.2) (layer "B.Cu") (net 7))
 (segment (start 134.62 74.93) (end 151.13 91.44) (width 0.2) (layer "F.Cu") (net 8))
 (segment (start 134.227 74.93) (end 134.62 74.93) (width 0.2) (layer "F.Cu") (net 8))
 (via (at 134.227 74.93) (size 0.6) (drill 0.3) (layers "F.Cu" "B.Cu") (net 8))
 (segment (start 119.0761 64.889) (end 124.186 64.889) (width 0.2) (layer "B.Cu") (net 8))
 (segment (start 115.3811 61.194) (end 119.0761 64.889) (width 0.2) (layer "B.Cu") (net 8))
 (segment (start 124.186 64.889) (end 134.227 74.93) (width 0.2) (layer "B.Cu") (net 8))
 (segment (start 100.965 47.139816) (end 115.019184 61.194) (width 0.2) (layer "B.Cu") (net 8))
 (segment (start 115.019184 61.194) (end 115.3811 61.194) (width 0.2) (layer "B.Cu") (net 8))
 (segment (start 100.965 45.085) (end 100.965 47.139816) (width 0.2) (layer "B.Cu") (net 8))
 (segment (start 86.509816 64.135) (end 106.748313 84.373497) (width 0.2) (layer "B.Cu") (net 5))
 (segment (start 147.527 85.297) (end 151.13 88.9) (width 0.2) (layer "B.Cu") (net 5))
 (segment (start 81.915 64.135) (end 86.509816 64.135) (width 0.2) (layer "B.Cu") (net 5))
 (segment (start 135.44969 85.297) (end 147.527 85.297) (width 0.2) (layer "B.Cu") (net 5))
 (segment (start 134.526187 84.373497) (end 135.44969 85.297) (width 0.2) (layer "B.Cu") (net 5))
 (segment (start 106.748313 84.373497) (end 134.526187 84.373497) (width 0.2) (layer "B.Cu") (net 5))
 (segment (start 130.26908 80.55092) (end 130.26908 78.037977) (width 0.2) (layer "F.Cu") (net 9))
 (segment (start 130.26908 78.037977) (end 133.978057 74.329) (width 0.2) (layer "F.Cu") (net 9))
 (segment (start 133.978057 74.329) (end 139.934 74.329) (width 0.2) (layer "F.Cu") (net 9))
 (segment (start 139.934 74.329) (end 151.965 86.36) (width 0.2) (layer "F.Cu") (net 9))
 (via (at 130.26908 80.55092) (size 0.6) (drill 0.3) (layers "F.Cu" "B.Cu") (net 9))
 (segment (start 100.965 66.189816) (end 115.185389 80.410205) (width 0.2) (layer "B.Cu") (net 9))
 (segment (start 130.409795 80.410205) (end 130.26908 80.55092) (width 0.2) (layer "B.Cu") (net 9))
 (segment (start 115.185389 80.410205) (end 130.409795 80.410205) (width 0.2) (layer "B.Cu") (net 9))
 (segment (start 100.965 64.135) (end 100.965 66.189816) (width 0.2) (layer "B.Cu") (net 9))
 (segment (start 118.85 42.8625) (end 121.452 45.4645) (width 0.2) (layer "B.Cu") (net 10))
 (segment (start 121.452 54.142) (end 151.13 83.82) (width 0.2) (layer "B.Cu") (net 10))
 (segment (start 121.452 45.4645) (end 121.452 54.142) (width 0.2) (layer "B.Cu") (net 10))
 (segment (start 150.68969 84.883) (end 151.57031 84.883) (width 0.2) (layer "B.Cu") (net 11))
 (segment (start 152.193 84.26031) (end 152.193 82.343) (width 0.2) (layer "B.Cu") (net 11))
 (segment (start 151.57031 84.883) (end 152.193 84.26031) (width 0.2) (layer "B.Cu") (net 11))
 (segment (start 118.85 53.04331) (end 150.68969 84.883) (width 0.2) (layer "B.Cu") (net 11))
 (segment (start 152.193 82.343) (end 151.13 81.28) (width 0.2) (layer "B.Cu") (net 11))
 (segment (start 118.85 47.8625) (end 118.85 53.04331) (width 0.2) (layer "B.Cu") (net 11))
 (segment (start 119.75 48.7625) (end 118.85 47.8625) (width 0.2) (layer "B.Cu") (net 11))
 (segment (start 134.827 82.757) (end 135.89 83.82) (width 0.2) (layer "B.Cu") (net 14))
 (segment (start 134.827 73.587) (end 134.827 82.757) (width 0.2) (layer "B.Cu") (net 14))
 (segment (start 119.66 58.42) (end 134.827 73.587) (width 0.2) (layer "B.Cu") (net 14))
 (segment (start 118.509 57.94324) (end 119.18324 57.269) (width 0.2) (layer "B.Cu") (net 15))
 (segment (start 119.18324 57.269) (end 120.13676 57.269) (width 0.2) (layer "B.Cu") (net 15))
 (segment (start 151.57031 89.963) (end 139.493 89.963) (width 0.2) (layer "B.Cu") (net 15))
 (segment (start 152.193 88.45969) (end 152.193 89.34031) (width 0.2) (layer "B.Cu") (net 15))
 (segment (start 120.13676 57.269) (end 150.70476 87.837) (width 0.2) (layer "B.Cu") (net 15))
 (segment (start 118.509 59.809) (end 118.509 57.94324) (width 0.2) (layer "B.Cu") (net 15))
 (segment (start 119.66 60.96) (end 118.509 59.809) (width 0.2) (layer "B.Cu") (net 15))
 (segment (start 150.70476 87.837) (end 151.57031 87.837) (width 0.2) (layer "B.Cu") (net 15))
 (segment (start 139.493 89.963) (end 135.89 86.36) (width 0.2) (layer "B.Cu") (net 15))
 (segment (start 152.193 89.34031) (end 151.57031 89.963) (width 0.2) (layer "B.Cu") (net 15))
 (segment (start 151.57031 87.837) (end 152.193 88.45969) (width 0.2) (layer "B.Cu") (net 15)))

